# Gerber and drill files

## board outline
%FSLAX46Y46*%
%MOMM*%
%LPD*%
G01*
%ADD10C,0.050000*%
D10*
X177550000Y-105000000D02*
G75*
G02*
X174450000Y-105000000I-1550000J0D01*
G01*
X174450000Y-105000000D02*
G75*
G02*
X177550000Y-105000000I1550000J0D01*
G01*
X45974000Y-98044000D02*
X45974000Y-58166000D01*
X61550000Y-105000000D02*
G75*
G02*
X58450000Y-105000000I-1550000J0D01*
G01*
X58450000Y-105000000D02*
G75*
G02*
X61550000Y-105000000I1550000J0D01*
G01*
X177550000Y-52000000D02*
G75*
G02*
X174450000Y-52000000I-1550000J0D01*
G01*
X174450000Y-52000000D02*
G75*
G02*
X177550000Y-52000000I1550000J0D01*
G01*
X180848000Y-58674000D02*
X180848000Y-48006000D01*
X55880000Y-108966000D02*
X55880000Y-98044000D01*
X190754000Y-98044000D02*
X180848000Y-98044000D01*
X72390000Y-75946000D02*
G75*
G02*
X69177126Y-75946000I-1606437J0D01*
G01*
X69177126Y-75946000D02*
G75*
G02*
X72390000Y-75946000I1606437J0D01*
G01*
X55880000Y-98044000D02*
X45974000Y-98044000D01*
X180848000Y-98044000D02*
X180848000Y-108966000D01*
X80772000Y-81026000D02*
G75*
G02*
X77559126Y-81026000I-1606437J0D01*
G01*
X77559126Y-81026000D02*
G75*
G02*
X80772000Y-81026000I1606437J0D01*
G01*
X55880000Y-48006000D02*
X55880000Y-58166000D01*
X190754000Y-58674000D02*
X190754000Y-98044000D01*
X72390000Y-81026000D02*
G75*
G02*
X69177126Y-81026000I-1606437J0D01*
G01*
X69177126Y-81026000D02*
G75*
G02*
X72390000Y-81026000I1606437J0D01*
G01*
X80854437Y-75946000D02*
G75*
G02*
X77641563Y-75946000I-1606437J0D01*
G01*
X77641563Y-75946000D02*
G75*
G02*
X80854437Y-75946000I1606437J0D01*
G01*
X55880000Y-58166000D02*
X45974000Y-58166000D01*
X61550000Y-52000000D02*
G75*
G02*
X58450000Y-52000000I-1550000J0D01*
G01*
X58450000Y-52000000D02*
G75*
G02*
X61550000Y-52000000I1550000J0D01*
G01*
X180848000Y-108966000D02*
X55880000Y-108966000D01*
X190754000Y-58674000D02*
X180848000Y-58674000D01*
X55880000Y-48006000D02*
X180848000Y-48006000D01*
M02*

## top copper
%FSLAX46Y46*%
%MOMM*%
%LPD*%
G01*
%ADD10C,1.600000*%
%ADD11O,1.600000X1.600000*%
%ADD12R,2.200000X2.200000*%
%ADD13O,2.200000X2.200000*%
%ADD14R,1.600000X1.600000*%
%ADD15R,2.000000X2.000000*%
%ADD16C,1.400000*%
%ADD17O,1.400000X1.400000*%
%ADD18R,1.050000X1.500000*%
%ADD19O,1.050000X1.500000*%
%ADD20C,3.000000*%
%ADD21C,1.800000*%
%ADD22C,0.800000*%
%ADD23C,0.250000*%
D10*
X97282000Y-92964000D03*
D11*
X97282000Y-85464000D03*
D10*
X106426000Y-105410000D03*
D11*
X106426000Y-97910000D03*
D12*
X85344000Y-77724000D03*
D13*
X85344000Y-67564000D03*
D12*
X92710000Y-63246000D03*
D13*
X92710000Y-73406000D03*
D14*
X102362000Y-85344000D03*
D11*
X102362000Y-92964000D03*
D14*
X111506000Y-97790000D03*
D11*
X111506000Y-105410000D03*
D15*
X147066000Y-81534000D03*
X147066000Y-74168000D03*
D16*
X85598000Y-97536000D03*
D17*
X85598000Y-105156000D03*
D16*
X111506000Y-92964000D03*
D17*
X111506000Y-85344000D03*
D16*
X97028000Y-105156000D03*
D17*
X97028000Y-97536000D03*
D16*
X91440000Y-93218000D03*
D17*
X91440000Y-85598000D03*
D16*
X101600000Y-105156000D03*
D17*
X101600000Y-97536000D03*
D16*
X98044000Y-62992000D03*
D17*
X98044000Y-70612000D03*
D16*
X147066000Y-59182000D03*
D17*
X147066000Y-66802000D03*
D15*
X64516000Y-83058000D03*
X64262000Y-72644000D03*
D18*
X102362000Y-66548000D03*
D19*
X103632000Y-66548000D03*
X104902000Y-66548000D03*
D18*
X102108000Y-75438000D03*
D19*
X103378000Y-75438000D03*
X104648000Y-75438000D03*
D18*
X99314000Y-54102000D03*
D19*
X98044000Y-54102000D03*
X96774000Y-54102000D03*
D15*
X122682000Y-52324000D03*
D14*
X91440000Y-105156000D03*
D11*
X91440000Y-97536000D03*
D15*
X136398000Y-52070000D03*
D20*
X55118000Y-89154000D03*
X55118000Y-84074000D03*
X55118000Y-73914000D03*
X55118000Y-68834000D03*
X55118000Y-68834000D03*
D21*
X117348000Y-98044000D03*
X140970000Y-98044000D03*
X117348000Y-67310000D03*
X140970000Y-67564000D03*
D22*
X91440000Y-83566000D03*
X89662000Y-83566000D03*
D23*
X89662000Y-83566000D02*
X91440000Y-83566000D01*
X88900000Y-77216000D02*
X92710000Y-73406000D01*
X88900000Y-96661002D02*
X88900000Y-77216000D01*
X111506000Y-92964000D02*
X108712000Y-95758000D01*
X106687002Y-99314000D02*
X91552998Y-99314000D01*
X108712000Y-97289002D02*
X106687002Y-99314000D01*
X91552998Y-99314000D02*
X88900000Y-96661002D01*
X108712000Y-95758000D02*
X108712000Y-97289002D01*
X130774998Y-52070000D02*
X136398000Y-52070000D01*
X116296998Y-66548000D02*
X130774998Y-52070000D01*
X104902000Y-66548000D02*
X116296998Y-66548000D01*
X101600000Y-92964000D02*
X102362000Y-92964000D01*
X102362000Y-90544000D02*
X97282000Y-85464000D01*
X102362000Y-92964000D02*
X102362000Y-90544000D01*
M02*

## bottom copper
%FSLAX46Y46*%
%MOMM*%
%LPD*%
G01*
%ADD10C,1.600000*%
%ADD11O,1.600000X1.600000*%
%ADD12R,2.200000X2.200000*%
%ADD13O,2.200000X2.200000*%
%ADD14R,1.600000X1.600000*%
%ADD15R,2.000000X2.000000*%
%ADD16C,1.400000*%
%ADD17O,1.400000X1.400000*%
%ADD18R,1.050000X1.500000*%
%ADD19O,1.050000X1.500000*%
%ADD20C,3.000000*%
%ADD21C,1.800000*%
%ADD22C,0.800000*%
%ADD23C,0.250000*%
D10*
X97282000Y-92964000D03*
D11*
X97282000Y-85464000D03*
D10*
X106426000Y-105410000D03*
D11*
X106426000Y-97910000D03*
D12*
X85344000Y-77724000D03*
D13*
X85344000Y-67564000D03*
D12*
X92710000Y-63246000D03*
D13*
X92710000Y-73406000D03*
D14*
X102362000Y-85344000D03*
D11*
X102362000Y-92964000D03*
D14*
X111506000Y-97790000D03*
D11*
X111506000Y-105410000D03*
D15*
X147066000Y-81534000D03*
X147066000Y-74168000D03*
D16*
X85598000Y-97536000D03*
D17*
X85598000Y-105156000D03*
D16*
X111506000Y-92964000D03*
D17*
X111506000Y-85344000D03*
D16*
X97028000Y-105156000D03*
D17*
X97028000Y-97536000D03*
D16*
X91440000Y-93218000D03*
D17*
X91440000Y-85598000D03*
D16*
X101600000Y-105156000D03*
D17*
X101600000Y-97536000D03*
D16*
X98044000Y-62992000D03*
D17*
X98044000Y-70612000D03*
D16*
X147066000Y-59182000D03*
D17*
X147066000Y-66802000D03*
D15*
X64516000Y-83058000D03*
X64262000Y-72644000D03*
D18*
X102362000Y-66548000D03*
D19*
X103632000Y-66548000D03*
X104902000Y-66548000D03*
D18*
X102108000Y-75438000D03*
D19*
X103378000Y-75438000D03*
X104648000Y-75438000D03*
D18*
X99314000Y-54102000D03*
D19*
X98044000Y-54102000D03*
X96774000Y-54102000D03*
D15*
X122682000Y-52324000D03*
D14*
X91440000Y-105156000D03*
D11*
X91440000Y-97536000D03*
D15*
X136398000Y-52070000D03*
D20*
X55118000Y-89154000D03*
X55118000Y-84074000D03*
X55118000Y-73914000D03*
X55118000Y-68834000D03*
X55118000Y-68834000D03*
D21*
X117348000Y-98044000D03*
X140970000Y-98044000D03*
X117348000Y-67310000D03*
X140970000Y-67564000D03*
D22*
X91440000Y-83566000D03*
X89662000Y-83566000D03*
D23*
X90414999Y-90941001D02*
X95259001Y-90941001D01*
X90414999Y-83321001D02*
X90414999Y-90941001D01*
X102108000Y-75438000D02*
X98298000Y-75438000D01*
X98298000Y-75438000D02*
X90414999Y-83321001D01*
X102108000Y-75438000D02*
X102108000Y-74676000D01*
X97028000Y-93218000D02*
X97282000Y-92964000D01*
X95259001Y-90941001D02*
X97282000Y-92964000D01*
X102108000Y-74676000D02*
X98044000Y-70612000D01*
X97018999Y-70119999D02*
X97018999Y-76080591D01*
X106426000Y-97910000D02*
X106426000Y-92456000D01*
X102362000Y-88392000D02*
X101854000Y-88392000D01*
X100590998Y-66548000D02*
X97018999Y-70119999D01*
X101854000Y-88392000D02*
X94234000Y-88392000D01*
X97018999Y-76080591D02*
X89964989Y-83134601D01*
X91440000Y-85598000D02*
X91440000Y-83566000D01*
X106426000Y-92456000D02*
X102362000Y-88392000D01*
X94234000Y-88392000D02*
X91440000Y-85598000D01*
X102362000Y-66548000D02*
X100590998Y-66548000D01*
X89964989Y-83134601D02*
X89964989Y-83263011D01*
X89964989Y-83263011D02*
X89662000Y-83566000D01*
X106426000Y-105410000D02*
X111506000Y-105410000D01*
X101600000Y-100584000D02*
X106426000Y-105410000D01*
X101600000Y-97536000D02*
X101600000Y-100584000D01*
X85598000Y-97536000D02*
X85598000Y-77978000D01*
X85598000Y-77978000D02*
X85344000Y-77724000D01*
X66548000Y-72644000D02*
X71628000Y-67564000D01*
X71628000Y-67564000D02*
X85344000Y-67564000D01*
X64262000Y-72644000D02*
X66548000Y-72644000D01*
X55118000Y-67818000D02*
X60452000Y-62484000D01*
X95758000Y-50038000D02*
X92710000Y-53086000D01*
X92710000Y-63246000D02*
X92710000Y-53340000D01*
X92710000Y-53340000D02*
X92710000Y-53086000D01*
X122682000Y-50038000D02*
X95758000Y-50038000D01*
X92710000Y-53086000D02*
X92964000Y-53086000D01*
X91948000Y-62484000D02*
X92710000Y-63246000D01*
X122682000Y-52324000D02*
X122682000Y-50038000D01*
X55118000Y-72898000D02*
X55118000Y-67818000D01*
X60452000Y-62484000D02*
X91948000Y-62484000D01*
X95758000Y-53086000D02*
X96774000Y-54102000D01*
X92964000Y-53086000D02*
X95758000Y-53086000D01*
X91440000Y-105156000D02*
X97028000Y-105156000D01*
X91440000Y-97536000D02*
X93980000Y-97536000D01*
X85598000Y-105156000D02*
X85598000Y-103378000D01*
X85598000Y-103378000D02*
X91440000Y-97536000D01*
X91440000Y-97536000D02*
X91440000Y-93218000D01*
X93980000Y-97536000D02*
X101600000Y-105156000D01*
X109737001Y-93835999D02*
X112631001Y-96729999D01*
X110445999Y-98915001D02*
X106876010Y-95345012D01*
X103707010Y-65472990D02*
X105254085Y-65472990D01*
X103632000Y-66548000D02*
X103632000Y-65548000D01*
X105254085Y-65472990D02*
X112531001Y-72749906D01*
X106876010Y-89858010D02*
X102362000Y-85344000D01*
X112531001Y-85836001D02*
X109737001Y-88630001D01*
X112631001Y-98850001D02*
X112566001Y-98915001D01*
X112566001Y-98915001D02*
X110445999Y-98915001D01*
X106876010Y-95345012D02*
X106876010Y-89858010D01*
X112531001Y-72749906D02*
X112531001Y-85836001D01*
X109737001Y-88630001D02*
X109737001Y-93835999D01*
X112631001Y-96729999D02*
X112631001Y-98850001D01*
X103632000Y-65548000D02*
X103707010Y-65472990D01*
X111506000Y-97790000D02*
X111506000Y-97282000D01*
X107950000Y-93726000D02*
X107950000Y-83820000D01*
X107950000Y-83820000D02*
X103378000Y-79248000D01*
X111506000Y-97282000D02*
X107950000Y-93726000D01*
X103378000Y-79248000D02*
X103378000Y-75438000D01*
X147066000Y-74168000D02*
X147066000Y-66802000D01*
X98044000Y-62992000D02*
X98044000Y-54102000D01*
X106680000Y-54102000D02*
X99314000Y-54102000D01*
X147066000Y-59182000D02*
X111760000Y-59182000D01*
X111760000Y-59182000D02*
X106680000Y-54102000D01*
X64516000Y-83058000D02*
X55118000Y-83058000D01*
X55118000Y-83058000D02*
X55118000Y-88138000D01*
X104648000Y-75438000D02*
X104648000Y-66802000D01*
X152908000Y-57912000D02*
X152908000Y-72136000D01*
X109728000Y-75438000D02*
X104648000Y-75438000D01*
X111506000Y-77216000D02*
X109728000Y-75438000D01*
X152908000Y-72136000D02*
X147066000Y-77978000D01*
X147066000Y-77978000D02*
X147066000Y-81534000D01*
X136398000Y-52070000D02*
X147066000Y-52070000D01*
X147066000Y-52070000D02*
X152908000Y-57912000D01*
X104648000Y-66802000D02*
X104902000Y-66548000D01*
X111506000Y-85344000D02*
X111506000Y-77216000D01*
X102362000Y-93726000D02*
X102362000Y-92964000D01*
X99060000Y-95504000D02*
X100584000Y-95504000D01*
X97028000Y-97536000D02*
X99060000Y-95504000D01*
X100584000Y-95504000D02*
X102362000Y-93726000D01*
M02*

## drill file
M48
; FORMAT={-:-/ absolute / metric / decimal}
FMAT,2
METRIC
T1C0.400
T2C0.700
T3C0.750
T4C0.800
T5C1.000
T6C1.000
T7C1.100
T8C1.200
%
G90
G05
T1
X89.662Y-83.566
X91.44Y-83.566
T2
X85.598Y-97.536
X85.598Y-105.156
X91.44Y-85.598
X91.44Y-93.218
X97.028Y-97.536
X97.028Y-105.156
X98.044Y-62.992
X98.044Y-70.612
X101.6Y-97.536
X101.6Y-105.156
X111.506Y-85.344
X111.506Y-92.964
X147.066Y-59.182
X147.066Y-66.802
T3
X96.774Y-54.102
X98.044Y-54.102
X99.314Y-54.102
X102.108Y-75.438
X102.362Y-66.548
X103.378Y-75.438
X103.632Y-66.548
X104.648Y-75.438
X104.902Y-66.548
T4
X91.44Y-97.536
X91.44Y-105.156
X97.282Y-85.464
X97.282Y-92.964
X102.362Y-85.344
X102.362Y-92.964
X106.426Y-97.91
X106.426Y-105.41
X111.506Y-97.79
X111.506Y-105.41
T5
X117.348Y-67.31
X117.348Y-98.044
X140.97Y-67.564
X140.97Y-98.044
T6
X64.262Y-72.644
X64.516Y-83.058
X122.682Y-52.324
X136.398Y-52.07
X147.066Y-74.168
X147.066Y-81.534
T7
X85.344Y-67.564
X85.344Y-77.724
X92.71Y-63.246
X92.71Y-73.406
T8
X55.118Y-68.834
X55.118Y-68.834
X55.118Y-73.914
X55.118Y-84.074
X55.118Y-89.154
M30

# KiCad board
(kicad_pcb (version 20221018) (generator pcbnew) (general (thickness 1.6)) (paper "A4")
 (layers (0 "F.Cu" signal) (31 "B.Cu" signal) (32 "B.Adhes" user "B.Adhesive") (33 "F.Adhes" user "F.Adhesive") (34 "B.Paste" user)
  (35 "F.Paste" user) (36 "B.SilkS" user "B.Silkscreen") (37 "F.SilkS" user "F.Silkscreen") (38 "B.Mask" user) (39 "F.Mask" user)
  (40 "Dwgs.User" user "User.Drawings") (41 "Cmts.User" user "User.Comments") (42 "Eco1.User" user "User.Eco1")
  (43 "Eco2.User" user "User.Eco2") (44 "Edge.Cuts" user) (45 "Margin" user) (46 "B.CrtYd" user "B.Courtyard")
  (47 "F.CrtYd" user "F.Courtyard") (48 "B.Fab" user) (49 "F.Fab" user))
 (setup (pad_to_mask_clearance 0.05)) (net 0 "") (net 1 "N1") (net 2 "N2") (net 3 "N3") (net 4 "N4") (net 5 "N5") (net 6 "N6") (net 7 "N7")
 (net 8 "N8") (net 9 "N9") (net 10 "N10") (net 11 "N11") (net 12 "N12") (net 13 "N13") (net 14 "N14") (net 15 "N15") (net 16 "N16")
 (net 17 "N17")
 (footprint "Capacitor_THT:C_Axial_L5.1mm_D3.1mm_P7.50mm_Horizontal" (layer "F.Cu") (at 97.282 92.964 90)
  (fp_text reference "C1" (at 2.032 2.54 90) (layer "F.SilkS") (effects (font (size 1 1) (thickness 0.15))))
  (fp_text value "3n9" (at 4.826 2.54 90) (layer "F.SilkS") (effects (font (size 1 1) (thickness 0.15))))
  (pad "1" thru_hole circle (at 0 0 90) (size 1.6 1.6) (drill 0.8) (layers "*.Cu" "*.Mask") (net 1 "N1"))
  (pad "2" thru_hole oval (at 7.5 0 90) (size 1.6 1.6) (drill 0.8) (layers "*.Cu" "*.Mask") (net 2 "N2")))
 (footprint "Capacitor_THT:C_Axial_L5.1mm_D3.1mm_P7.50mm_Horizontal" (layer "F.Cu") (at 106.426 105.41 90)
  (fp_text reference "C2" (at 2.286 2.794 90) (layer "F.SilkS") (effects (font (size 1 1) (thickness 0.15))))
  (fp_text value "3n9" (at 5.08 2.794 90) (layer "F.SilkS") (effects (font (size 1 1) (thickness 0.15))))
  (pad "1" thru_hole circle (at 0 0 90) (size 1.6 1.6) (drill 0.8) (layers "*.Cu" "*.Mask") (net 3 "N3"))
  (pad "2" thru_hole oval (at 7.5 0 90) (size 1.6 1.6) (drill 0.8) (layers "*.Cu" "*.Mask") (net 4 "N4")))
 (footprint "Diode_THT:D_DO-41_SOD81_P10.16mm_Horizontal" (layer "F.Cu") (at 85.344 77.724 90)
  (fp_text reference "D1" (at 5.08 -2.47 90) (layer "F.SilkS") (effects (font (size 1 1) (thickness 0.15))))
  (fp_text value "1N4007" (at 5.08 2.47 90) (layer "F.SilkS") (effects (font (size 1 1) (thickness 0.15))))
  (pad "1" thru_hole rect (at 0 0 90) (size 2.2 2.2) (drill 1.1) (layers "*.Cu" "*.Mask") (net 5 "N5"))
  (pad "2" thru_hole oval (at 10.16 0 90) (size 2.2 2.2) (drill 1.1) (layers "*.Cu" "*.Mask") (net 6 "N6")))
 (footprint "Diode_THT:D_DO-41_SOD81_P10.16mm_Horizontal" (layer "F.Cu") (at 92.71 63.246 -90)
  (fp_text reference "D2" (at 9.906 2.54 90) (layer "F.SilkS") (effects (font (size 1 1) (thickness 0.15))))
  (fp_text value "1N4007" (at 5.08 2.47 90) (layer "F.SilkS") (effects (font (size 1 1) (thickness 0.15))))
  (pad "1" thru_hole rect (at 0 0 270) (size 2.2 2.2) (drill 1.1) (layers "*.Cu" "*.Mask") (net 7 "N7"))
  (pad "2" thru_hole oval (at 10.16 0 270) (size 2.2 2.2) (drill 1.1) (layers "*.Cu" "*.Mask") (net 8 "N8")))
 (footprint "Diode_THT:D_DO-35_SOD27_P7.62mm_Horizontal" (layer "F.Cu") (at 102.362 85.344 -90)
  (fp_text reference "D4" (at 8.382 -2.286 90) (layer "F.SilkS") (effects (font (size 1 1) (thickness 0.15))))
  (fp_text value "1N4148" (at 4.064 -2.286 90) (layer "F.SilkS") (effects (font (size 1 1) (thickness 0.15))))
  (pad "1" thru_hole rect (at 0 0 270) (size 1.6 1.6) (drill 0.8) (layers "*.Cu" "*.Mask") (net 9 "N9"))
  (pad "2" thru_hole oval (at 7.62 0 270) (size 1.6 1.6) (drill 0.8) (layers "*.Cu" "*.Mask") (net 2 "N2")))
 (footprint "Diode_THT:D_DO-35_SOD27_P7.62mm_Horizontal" (layer "F.Cu") (at 111.506 97.79 -90)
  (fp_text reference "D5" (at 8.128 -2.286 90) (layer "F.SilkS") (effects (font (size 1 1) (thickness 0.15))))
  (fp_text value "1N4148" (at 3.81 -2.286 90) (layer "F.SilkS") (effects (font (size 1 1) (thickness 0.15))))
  (pad "1" thru_hole rect (at 0 0 270) (size 1.6 1.6) (drill 0.8) (layers "*.Cu" "*.Mask") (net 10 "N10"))
  (pad "2" thru_hole oval (at 7.62 0 270) (size 1.6 1.6) (drill 0.8) (layers "*.Cu" "*.Mask") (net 3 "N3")))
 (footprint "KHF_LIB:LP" (layer "F.Cu") (at 147.066 81.534)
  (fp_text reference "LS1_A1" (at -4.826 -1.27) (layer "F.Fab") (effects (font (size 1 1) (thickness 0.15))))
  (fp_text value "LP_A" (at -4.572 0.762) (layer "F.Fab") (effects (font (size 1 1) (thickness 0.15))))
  (pad "1" thru_hole rect (at 0 0) (size 2 2) (drill 1) (layers "*.Cu" "*.Mask") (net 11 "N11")))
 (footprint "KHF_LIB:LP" (layer "F.Cu") (at 147.066 74.168)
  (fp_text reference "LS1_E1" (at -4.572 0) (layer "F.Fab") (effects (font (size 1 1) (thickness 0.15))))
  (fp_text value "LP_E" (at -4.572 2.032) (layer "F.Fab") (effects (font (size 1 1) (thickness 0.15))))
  (pad "1" thru_hole rect (at 0 0) (size 2 2) (drill 1) (layers "*.Cu" "*.Mask") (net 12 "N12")))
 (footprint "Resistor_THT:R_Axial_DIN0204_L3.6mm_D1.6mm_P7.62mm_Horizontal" (layer "F.Cu") (at 85.598 97.536 -90)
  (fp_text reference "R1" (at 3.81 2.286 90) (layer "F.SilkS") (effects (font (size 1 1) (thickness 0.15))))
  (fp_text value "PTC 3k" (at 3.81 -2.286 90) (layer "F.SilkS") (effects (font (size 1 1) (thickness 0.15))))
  (pad "1" thru_hole circle (at 0 0 270) (size 1.4 1.4) (drill 0.7) (layers "*.Cu" "*.Mask") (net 5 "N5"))
  (pad "2" thru_hole oval (at 7.62 0 270) (size 1.4 1.4) (drill 0.7) (layers "*.Cu" "*.Mask") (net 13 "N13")))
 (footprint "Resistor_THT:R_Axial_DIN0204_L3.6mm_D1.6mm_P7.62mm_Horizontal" (layer "F.Cu") (at 111.506 92.964 90)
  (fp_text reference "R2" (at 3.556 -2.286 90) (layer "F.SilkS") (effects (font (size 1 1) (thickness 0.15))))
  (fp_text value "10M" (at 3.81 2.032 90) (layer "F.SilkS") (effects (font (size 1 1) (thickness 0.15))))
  (pad "1" thru_hole circle (at 0 0 90) (size 1.4 1.4) (drill 0.7) (layers "*.Cu" "*.Mask") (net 8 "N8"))
  (pad "2" thru_hole oval (at 7.62 0 90) (size 1.4 1.4) (drill 0.7) (layers "*.Cu" "*.Mask") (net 11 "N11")))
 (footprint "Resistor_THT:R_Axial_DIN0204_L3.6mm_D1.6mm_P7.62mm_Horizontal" (layer "F.Cu") (at 97.028 105.156 90)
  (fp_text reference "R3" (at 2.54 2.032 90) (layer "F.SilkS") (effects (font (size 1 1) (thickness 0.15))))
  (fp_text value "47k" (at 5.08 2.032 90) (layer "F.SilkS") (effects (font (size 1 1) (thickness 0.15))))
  (pad "1" thru_hole circle (at 0 0 90) (size 1.4 1.4) (drill 0.7) (layers "*.Cu" "*.Mask") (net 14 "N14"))
  (pad "2" thru_hole oval (at 7.62 0 90) (size 1.4 1.4) (drill 0.7) (layers "*.Cu" "*.Mask") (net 2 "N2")))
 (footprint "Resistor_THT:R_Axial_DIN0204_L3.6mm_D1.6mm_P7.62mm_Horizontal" (layer "F.Cu") (at 91.44 93.218 90)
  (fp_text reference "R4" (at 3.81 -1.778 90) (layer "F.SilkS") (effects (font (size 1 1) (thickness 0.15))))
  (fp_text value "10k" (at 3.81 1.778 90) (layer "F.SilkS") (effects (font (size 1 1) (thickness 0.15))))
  (pad "1" thru_hole circle (at 0 0 90) (size 1.4 1.4) (drill 0.7) (layers "*.Cu" "*.Mask") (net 13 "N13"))
  (pad "2" thru_hole oval (at 7.62 0 90) (size 1.4 1.4) (drill 0.7) (layers "*.Cu" "*.Mask") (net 4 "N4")))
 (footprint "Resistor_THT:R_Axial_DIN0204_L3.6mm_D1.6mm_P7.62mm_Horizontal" (layer "F.Cu") (at 101.6 105.156 90)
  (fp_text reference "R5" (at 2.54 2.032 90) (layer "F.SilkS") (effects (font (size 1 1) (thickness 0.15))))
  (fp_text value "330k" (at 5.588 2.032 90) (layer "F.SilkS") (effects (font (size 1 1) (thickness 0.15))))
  (pad "1" thru_hole circle (at 0 0 90) (size 1.4 1.4) (drill 0.7) (layers "*.Cu" "*.Mask") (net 13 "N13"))
  (pad "2" thru_hole oval (at 7.62 0 90) (size 1.4 1.4) (drill 0.7) (layers "*.Cu" "*.Mask") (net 3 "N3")))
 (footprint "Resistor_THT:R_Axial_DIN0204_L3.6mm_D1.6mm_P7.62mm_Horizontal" (layer "F.Cu") (at 98.044 62.992 -90)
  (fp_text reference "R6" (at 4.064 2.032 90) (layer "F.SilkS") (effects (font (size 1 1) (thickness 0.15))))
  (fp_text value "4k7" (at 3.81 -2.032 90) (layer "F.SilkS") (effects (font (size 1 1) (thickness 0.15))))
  (pad "1" thru_hole circle (at 0 0 270) (size 1.4 1.4) (drill 0.7) (layers "*.Cu" "*.Mask") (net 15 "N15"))
  (pad "2" thru_hole oval (at 7.62 0 270) (size 1.4 1.4) (drill 0.7) (layers "*.Cu" "*.Mask") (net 1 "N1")))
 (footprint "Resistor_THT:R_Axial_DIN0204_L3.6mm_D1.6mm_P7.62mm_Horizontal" (layer "F.Cu") (at 147.066 59.182 -90)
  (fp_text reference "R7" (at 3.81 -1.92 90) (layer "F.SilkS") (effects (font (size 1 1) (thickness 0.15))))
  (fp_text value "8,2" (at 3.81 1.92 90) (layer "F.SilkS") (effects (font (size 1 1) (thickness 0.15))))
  (pad "1" thru_hole circle (at 0 0 270) (size 1.4 1.4) (drill 0.7) (layers "*.Cu" "*.Mask") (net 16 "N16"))
  (pad "2" thru_hole oval (at 7.62 0 270) (size 1.4 1.4) (drill 0.7) (layers "*.Cu" "*.Mask") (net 12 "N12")))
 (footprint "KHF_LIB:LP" (layer "F.Cu") (at 64.516 83.058)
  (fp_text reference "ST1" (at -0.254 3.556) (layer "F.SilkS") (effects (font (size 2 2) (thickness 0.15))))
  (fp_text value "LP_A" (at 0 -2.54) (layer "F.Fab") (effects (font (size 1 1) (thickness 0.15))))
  (pad "1" thru_hole rect (at 0 0) (size 2 2) (drill 1) (layers "*.Cu" "*.Mask") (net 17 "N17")))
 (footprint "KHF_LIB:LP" (layer "F.Cu") (at 64.262 72.644)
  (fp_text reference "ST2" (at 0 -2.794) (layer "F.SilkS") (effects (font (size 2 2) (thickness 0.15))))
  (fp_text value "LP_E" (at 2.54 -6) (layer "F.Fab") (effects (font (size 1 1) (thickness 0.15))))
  (pad "1" thru_hole rect (at 0 0) (size 2 2) (drill 1) (layers "*.Cu" "*.Mask") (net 6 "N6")))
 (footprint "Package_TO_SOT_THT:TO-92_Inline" (layer "F.Cu") (at 102.362 66.548)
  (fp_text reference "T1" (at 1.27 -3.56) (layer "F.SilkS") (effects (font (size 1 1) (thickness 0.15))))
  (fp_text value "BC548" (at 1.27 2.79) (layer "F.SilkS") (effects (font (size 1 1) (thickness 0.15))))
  (pad "1" thru_hole rect (at 0 0) (size 1.05 1.5) (drill 0.75) (layers "*.Cu" "*.Mask") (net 4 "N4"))
  (pad "2" thru_hole oval (at 1.27 0) (size 1.05 1.5) (drill 0.75) (layers "*.Cu" "*.Mask") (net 9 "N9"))
  (pad "3" thru_hole oval (at 2.54 0) (size 1.05 1.5) (drill 0.75) (layers "*.Cu" "*.Mask") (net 11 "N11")))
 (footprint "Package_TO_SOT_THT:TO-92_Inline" (layer "F.Cu") (at 102.108 75.438)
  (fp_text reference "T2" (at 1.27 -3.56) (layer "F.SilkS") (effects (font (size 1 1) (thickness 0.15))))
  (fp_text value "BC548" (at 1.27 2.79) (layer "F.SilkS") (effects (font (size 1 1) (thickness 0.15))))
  (pad "1" thru_hole rect (at 0 0) (size 1.05 1.5) (drill 0.75) (layers "*.Cu" "*.Mask") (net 1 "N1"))
  (pad "2" thru_hole oval (at 1.27 0) (size 1.05 1.5) (drill 0.75) (layers "*.Cu" "*.Mask") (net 10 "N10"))
  (pad "3" thru_hole oval (at 2.54 0) (size 1.05 1.5) (drill 0.75) (layers "*.Cu" "*.Mask") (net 11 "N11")))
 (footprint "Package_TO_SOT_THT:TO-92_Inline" (layer "F.Cu") (at 99.314 54.102 180)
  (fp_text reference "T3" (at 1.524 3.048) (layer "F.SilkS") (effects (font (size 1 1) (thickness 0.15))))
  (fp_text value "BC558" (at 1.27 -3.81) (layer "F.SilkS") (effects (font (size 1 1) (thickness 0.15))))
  (pad "1" thru_hole rect (at 0 0 180) (size 1.05 1.5) (drill 0.75) (layers "*.Cu" "*.Mask") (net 16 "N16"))
  (pad "2" thru_hole oval (at 1.27 0 180) (size 1.05 1.5) (drill 0.75) (layers "*.Cu" "*.Mask") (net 15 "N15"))
  (pad "3" thru_hole oval (at 2.54 0 180) (size 1.05 1.5) (drill 0.75) (layers "*.Cu" "*.Mask") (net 7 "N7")))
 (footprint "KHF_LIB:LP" (layer "F.Cu") (at 122.682 52.324)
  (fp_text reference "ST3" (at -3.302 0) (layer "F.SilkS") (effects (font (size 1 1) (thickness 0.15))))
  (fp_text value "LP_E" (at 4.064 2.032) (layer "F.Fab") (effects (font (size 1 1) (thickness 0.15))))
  (pad "1" thru_hole rect (at 0 0) (size 2 2) (drill 1) (layers "*.Cu" "*.Mask") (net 7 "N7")))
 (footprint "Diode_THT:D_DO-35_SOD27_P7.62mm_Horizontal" (layer "F.Cu") (at 91.44 105.156 90)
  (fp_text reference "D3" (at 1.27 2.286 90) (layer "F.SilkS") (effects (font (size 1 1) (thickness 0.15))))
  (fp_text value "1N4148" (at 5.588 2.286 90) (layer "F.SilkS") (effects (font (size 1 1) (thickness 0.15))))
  (pad "1" thru_hole rect (at 0 0 90) (size 1.6 1.6) (drill 0.8) (layers "*.Cu" "*.Mask") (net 14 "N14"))
  (pad "2" thru_hole oval (at 7.62 0 90) (size 1.6 1.6) (drill 0.8) (layers "*.Cu" "*.Mask") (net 13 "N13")))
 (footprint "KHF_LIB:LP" (layer "F.Cu") (at 136.398 52.07)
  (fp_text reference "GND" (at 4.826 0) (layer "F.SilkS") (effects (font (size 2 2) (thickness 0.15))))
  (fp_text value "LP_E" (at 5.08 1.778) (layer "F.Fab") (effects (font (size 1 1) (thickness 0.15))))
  (pad "1" thru_hole rect (at 0 0) (size 2 2) (drill 1) (layers "*.Cu" "*.Mask") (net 11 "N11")))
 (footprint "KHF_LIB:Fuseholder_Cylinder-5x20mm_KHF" (layer "F.Cu") (at 55.118 89.154 90)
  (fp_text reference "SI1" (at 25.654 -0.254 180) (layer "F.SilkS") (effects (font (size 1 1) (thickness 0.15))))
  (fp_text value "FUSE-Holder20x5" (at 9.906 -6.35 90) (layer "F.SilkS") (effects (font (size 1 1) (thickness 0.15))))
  (pad "1" thru_hole circle (at 0 0 90) (size 3 3) (drill 1.2) (layers "*.Cu" "*.Mask") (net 17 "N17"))
  (pad "1" thru_hole circle (at 5.08 0 90) (size 3 3) (drill 1.2) (layers "*.Cu" "*.Mask") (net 17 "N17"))
  (pad "2" thru_hole circle (at 15.24 0 90) (size 3 3) (drill 1.2) (layers "*.Cu" "*.Mask") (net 7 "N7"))
  (pad "2" thru_hole circle (at 20.32 0 90) (size 3 3) (drill 1.2) (layers "*.Cu" "*.Mask") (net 7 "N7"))
  (pad "2" thru_hole circle (at 20.32 0 90) (size 3 3) (drill 1.2) (layers "*.Cu" "*.Mask") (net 7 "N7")))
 (gr_circle (center 176 105) (end 177.55 105) (stroke (width 0.05) (type solid)) (fill none) (layer "Edge.Cuts"))
 (gr_line (start 45.974 98.044) (end 45.974 58.166) (stroke (width 0.05) (type solid)) (layer "Edge.Cuts"))
 (gr_circle (center 60 105) (end 61.55 105) (stroke (width 0.05) (type solid)) (fill none) (layer "Edge.Cuts"))
 (gr_circle (center 176 52) (end 177.55 52) (stroke (width 0.05) (type solid)) (fill none) (layer "Edge.Cuts"))
 (gr_line (start 180.848 58.674) (end 180.848 48.006) (stroke (width 0.05) (type solid)) (layer "Edge.Cuts"))
 (gr_line (start 55.88 108.966) (end 55.88 98.044) (stroke (width 0.05) (type solid)) (layer "Edge.Cuts"))
 (gr_line (start 190.754 98.044) (end 180.848 98.044) (stroke (width 0.05) (type solid)) (layer "Edge.Cuts"))
 (gr_circle (center 70.783563 75.946) (end 69.259563 75.438) (stroke (width 0.05) (type solid)) (fill none) (layer "Edge.Cuts"))
 (gr_line (start 55.88 98.044) (end 45.974 98.044) (stroke (width 0.05) (type solid)) (layer "Edge.Cuts"))
 (gr_line (start 180.848 98.044) (end 180.848 108.966) (stroke (width 0.05) (type solid)) (layer "Edge.Cuts"))
 (gr_circle (center 79.165563 81.026) (end 77.641563 80.518) (stroke (width 0.05) (type solid)) (fill none) (layer "Edge.Cuts"))
 (gr_line (start 55.88 48.006) (end 55.88 58.166) (stroke (width 0.05) (type solid)) (layer "Edge.Cuts"))
 (gr_line (start 190.754 58.674) (end 190.754 98.044) (stroke (width 0.05) (type solid)) (layer "Edge.Cuts"))
 (gr_circle (center 70.783563 81.026) (end 69.259563 80.518) (stroke (width 0.05) (type solid)) (fill none) (layer "Edge.Cuts"))
 (gr_circle (center 79.248 75.946) (end 77.724 75.438) (stroke (width 0.05) (type solid)) (fill none) (layer "Edge.Cuts"))
 (gr_line (start 55.88 58.166) (end 45.974 58.166) (stroke (width 0.05) (type solid)) (layer "Edge.Cuts"))
 (gr_circle (center 60 52) (end 61.55 52) (stroke (width 0.05) (type solid)) (fill none) (layer "Edge.Cuts"))
 (gr_line (start 180.848 108.966) (end 55.88 108.966) (stroke (width 0.05) (type solid)) (layer "Edge.Cuts"))
 (gr_line (start 190.754 58.674) (end 180.848 58.674) (stroke (width 0.05) (type solid)) (layer "Edge.Cuts"))
 (gr_line (start 55.88 48.006) (end 180.848 48.006) (stroke (width 0.05) (type solid)) (layer "Edge.Cuts"))
 (via (at 117.348 98.044) (size 1.8) (drill 1) (layers "F.Cu" "B.Cu") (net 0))
 (via (at 140.97 98.044) (size 1.8) (drill 1) (layers "F.Cu" "B.Cu") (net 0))
 (via (at 117.348 67.31) (size 1.8) (drill 1) (layers "F.Cu" "B.Cu") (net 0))
 (via (at 140.97 67.564) (size 1.8) (drill 1) (layers "F.Cu" "B.Cu") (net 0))
 (segment (start 90.414999 90.941001) (end 95.259001 90.941001) (width 0.25) (layer "B.Cu") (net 1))
 (segment (start 90.414999 83.321001) (end 90.414999 90.941001) (width 0.25) (layer "B.Cu") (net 1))
 (segment (start 102.108 75.438) (end 98.298 75.438) (width 0.25) (layer "B.Cu") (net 1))
 (segment (start 98.298 75.438) (end 90.414999 83.321001) (width 0.25) (layer "B.Cu") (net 1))
 (segment (start 102.108 75.438) (end 102.108 74.676) (width 0.25) (layer "B.Cu") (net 1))
 (segment (start 97.028 93.218) (end 97.282 92.964) (width 0.25) (layer "B.Cu") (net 1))
 (segment (start 95.259001 90.941001) (end 97.282 92.964) (width 0.25) (layer "B.Cu") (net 1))
 (segment (start 102.108 74.676) (end 98.044 70.612) (width 0.25) (layer "B.Cu") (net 1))
 (segment (start 89.662 83.566) (end 91.44 83.566) (width 0.25) (layer "F.Cu") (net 4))
 (via (at 91.44 83.566) (size 0.8) (drill 0.4) (layers "F.Cu" "B.Cu") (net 4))
 (via (at 89.662 83.566) (size 0.8) (drill 0.4) (layers "F.Cu" "B.Cu") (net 4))
 (segment (start 97.018999 70.119999) (end 97.018999 76.080591) (width 0.25) (layer "B.Cu") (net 4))
 (segment (start 106.426 97.91) (end 106.426 92.456) (width 0.25) (layer "B.Cu") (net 4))
 (segment (start 102.362 88.392) (end 101.854 88.392) (width 0.25) (layer "B.Cu") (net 4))
 (segment (start 100.590998 66.548) (end 97.018999 70.119999) (width 0.25) (layer "B.Cu") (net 4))
 (segment (start 101.854 88.392) (end 94.234 88.392) (width 0.25) (layer "B.Cu") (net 4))
 (segment (start 97.018999 76.080591) (end 89.964989 83.134601) (width 0.25) (layer "B.Cu") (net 4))
 (segment (start 91.44 85.598) (end 91.44 83.566) (width 0.25) (layer "B.Cu") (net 4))
 (segment (start 106.426 92.456) (end 102.362 88.392) (width 0.25) (layer "B.Cu") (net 4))
 (segment (start 94.234 88.392) (end 91.44 85.598) (width 0.25) (layer "B.Cu") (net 4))
 (segment (start 102.362 66.548) (end 100.590998 66.548) (width 0.25) (layer "B.Cu") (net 4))
 (segment (start 89.964989 83.134601) (end 89.964989 83.263011) (width 0.25) (layer "B.Cu") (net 4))
 (segment (start 89.964989 83.263011) (end 89.662 83.566) (width 0.25) (layer "B.Cu") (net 4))
 (segment (start 106.426 105.41) (end 111.506 105.41) (width 0.25) (layer "B.Cu") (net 3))
 (segment (start 101.6 100.584) (end 106.426 105.41) (width 0.25) (layer "B.Cu") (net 3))
 (segment (start 101.6 97.536) (end 101.6 100.584) (width 0.25) (layer "B.Cu") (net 3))
 (segment (start 85.598 97.536) (end 85.598 77.978) (width 0.25) (layer "B.Cu") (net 5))
 (segment (start 85.598 77.978) (end 85.344 77.724) (width 0.25) (layer "B.Cu") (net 5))
 (segment (start 66.548 72.644) (end 71.628 67.564) (width 0.25) (layer "B.Cu") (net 6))
 (segment (start 71.628 67.564) (end 85.344 67.564) (width 0.25) (layer "B.Cu") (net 6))
 (segment (start 64.262 72.644) (end 66.548 72.644) (width 0.25) (layer "B.Cu") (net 6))
 (segment (start 88.9 77.216) (end 92.71 73.406) (width 0.25) (layer "F.Cu") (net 8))
 (segment (start 88.9 96.661002) (end 88.9 77.216) (width 0.25) (layer "F.Cu") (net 8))
 (segment (start 111.506 92.964) (end 108.712 95.758) (width 0.25) (layer "F.Cu") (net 8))
 (segment (start 106.687002 99.314) (end 91.552998 99.314) (width 0.25) (layer "F.Cu") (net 8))
 (segment (start 108.712 97.289002) (end 106.687002 99.314) (width 0.25) (layer "F.Cu") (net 8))
 (segment (start 91.552998 99.314) (end 88.9 96.661002) (width 0.25) (layer "F.Cu") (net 8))
 (segment (start 108.712 95.758) (end 108.712 97.289002) (width 0.25) (layer "F.Cu") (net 8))
 (segment (start 55.118 67.818) (end 60.452 62.484) (width 0.25) (layer "B.Cu") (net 7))
 (segment (start 95.758 50.038) (end 92.71 53.086) (width 0.25) (layer "B.Cu") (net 7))
 (segment (start 92.71 63.246) (end 92.71 53.34) (width 0.25) (layer "B.Cu") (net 7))
 (segment (start 92.71 53.34) (end 92.71 53.086) (width 0.25) (layer "B.Cu") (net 7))
 (segment (start 122.682 50.038) (end 95.758 50.038) (width 0.25) (layer "B.Cu") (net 7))
 (segment (start 92.71 53.086) (end 92.964 53.086) (width 0.25) (layer "B.Cu") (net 7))
 (segment (start 91.948 62.484) (end 92.71 63.246) (width 0.25) (layer "B.Cu") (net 7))
 (segment (start 122.682 52.324) (end 122.682 50.038) (width 0.25) (layer "B.Cu") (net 7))
 (segment (start 55.118 72.898) (end 55.118 67.818) (width 0.25) (layer "B.Cu") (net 7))
 (segment (start 60.452 62.484) (end 91.948 62.484) (width 0.25) (layer "B.Cu") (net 7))
 (segment (start 95.758 53.086) (end 96.774 54.102) (width 0.25) (layer "B.Cu") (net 7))
 (segment (start 92.964 53.086) (end 95.758 53.086) (width 0.25) (layer "B.Cu") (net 7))
 (segment (start 91.44 105.156) (end 97.028 105.156) (width 0.25) (layer "B.Cu") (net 14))
 (segment (start 91.44 97.536) (end 93.98 97.536) (width 0.25) (layer "B.Cu") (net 13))
 (segment (start 85.598 105.156) (end 85.598 103.378) (width 0.25) (layer "B.Cu") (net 13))
 (segment (start 85.598 103.378) (end 91.44 97.536) (width 0.25) (layer "B.Cu") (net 13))
 (segment (start 91.44 97.536) (end 91.44 93.218) (width 0.25) (layer "B.Cu") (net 13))
 (segment (start 93.98 97.536) (end 101.6 105.156) (width 0.25) (layer "B.Cu") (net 13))
 (segment (start 109.737001 93.835999) (end 112.631001 96.729999) (width 0.25) (layer "B.Cu") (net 9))
 (segment (start 110.445999 98.915001) (end 106.87601 95.345012) (width 0.25) (layer "B.Cu") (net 9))
 (segment (start 103.70701 65.47299) (end 105.254085 65.47299) (width 0.25) (layer "B.Cu") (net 9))
 (segment (start 103.632 66.548) (end 103.632 65.548) (width 0.25) (layer "B.Cu") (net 9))
 (segment (start 105.254085 65.47299) (end 112.531001 72.749906) (width 0.25) (layer "B.Cu") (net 9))
 (segment (start 106.87601 89.85801) (end 102.362 85.344) (width 0.25) (layer "B.Cu") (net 9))
 (segment (start 112.531001 85.836001) (end 109.737001 88.630001) (width 0.25) (layer "B.Cu") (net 9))
 (segment (start 112.631001 98.850001) (end 112.566001 98.915001) (width 0.25) (layer "B.Cu") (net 9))
 (segment (start 112.566001 98.915001) (end 110.445999 98.915001) (width 0.25) (layer "B.Cu") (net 9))
 (segment (start 106.87601 95.345012) (end 106.87601 89.85801) (width 0.25) (layer "B.Cu") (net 9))
 (segment (start 112.531001 72.749906) (end 112.531001 85.836001) (width 0.25) (layer "B.Cu") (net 9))
 (segment (start 109.737001 88.630001) (end 109.737001 93.835999) (width 0.25) (layer "B.Cu") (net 9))
 (segment (start 112.631001 96.729999) (end 112.631001 98.850001) (width 0.25) (layer "B.Cu") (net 9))
 (segment (start 103.632 65.548) (end 103.70701 65.47299) (width 0.25) (layer "B.Cu") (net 9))
 (segment (start 111.506 97.79) (end 111.506 97.282) (width 0.25) (layer "B.Cu") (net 10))
 (segment (start 107.95 93.726) (end 107.95 83.82) (width 0.25) (layer "B.Cu") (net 10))
 (segment (start 107.95 83.82) (end 103.378 79.248) (width 0.25) (layer "B.Cu") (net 10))
 (segment (start 111.506 97.282) (end 107.95 93.726) (width 0.25) (layer "B.Cu") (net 10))
 (segment (start 103.378 79.248) (end 103.378 75.438) (width 0.25) (layer "B.Cu") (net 10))
 (segment (start 147.066 74.168) (end 147.066 66.802) (width 0.25) (layer "B.Cu") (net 12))
 (segment (start 98.044 62.992) (end 98.044 54.102) (width 0.25) (layer "B.Cu") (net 15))
 (segment (start 106.68 54.102) (end 99.314 54.102) (width 0.25) (layer "B.Cu") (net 16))
 (segment (start 147.066 59.182) (end 111.76 59.182) (width 0.25) (layer "B.Cu") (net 16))
 (segment (start 111.76 59.182) (end 106.68 54.102) (width 0.25) (layer "B.Cu") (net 16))
 (segment (start 64.516 83.058) (end 55.118 83.058) (width 0.25) (layer "B.Cu") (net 17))
 (segment (start 55.118 83.058) (end 55.118 88.138) (width 0.25) (layer "B.Cu") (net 17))
 (segment (start 130.774998 52.07) (end 136.398 52.07) (width 0.25) (layer "F.Cu") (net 11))
 (segment (start 116.296998 66.548) (end 130.774998 52.07) (width 0.25) (layer "F.Cu") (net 11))
 (segment (start 104.902 66.548) (end 116.296998 66.548) (width 0.25) (layer "F.Cu") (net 11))
 (segment (start 104.648 75.438) (end 104.648 66.802) (width 0.25) (layer "B.Cu") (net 11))
 (segment (start 152.908 57.912) (end 152.908 72.136) (width 0.25) (layer "B.Cu") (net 11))
 (segment (start 109.728 75.438) (end 104.648 75.438) (width 0.25) (layer "B.Cu") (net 11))
 (segment (start 111.506 77.216) (end 109.728 75.438) (width 0.25) (layer "B.Cu") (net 11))
 (segment (start 152.908 72.136) (end 147.066 77.978) (width 0.25) (layer "B.Cu") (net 11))
 (segment (start 147.066 77.978) (end 147.066 81.534) (width 0.25) (layer "B.Cu") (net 11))
 (segment (start 136.398 52.07) (end 147.066 52.07) (width 0.25) (layer "B.Cu") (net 11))
 (segment (start 147.066 52.07) (end 152.908 57.912) (width 0.25) (layer "B.Cu") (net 11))
 (segment (start 104.648 66.802) (end 104.902 66.548) (width 0.25) (layer "B.Cu") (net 11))
 (segment (start 111.506 85.344) (end 111.506 77.216) (width 0.25) (layer "B.Cu") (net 11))
 (segment (start 101.6 92.964) (end 102.362 92.964) (width 0.25) (layer "F.Cu") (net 2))
 (segment (start 102.362 90.544) (end 97.282 85.464) (width 0.25) (layer "F.Cu") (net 2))
 (segment (start 102.362 92.964) (end 102.362 90.544) (width 0.25) (layer "F.Cu") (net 2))
 (segment (start 102.362 93.726) (end 102.362 92.964) (width 0.25) (layer "B.Cu") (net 2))
 (segment (start 99.06 95.504) (end 100.584 95.504) (width 0.25) (layer "B.Cu") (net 2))
 (segment (start 97.028 97.536) (end 99.06 95.504) (width 0.25) (layer "B.Cu") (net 2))
 (segment (start 100.584 95.504) (end 102.362 93.726) (width 0.25) (layer "B.Cu") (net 2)))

